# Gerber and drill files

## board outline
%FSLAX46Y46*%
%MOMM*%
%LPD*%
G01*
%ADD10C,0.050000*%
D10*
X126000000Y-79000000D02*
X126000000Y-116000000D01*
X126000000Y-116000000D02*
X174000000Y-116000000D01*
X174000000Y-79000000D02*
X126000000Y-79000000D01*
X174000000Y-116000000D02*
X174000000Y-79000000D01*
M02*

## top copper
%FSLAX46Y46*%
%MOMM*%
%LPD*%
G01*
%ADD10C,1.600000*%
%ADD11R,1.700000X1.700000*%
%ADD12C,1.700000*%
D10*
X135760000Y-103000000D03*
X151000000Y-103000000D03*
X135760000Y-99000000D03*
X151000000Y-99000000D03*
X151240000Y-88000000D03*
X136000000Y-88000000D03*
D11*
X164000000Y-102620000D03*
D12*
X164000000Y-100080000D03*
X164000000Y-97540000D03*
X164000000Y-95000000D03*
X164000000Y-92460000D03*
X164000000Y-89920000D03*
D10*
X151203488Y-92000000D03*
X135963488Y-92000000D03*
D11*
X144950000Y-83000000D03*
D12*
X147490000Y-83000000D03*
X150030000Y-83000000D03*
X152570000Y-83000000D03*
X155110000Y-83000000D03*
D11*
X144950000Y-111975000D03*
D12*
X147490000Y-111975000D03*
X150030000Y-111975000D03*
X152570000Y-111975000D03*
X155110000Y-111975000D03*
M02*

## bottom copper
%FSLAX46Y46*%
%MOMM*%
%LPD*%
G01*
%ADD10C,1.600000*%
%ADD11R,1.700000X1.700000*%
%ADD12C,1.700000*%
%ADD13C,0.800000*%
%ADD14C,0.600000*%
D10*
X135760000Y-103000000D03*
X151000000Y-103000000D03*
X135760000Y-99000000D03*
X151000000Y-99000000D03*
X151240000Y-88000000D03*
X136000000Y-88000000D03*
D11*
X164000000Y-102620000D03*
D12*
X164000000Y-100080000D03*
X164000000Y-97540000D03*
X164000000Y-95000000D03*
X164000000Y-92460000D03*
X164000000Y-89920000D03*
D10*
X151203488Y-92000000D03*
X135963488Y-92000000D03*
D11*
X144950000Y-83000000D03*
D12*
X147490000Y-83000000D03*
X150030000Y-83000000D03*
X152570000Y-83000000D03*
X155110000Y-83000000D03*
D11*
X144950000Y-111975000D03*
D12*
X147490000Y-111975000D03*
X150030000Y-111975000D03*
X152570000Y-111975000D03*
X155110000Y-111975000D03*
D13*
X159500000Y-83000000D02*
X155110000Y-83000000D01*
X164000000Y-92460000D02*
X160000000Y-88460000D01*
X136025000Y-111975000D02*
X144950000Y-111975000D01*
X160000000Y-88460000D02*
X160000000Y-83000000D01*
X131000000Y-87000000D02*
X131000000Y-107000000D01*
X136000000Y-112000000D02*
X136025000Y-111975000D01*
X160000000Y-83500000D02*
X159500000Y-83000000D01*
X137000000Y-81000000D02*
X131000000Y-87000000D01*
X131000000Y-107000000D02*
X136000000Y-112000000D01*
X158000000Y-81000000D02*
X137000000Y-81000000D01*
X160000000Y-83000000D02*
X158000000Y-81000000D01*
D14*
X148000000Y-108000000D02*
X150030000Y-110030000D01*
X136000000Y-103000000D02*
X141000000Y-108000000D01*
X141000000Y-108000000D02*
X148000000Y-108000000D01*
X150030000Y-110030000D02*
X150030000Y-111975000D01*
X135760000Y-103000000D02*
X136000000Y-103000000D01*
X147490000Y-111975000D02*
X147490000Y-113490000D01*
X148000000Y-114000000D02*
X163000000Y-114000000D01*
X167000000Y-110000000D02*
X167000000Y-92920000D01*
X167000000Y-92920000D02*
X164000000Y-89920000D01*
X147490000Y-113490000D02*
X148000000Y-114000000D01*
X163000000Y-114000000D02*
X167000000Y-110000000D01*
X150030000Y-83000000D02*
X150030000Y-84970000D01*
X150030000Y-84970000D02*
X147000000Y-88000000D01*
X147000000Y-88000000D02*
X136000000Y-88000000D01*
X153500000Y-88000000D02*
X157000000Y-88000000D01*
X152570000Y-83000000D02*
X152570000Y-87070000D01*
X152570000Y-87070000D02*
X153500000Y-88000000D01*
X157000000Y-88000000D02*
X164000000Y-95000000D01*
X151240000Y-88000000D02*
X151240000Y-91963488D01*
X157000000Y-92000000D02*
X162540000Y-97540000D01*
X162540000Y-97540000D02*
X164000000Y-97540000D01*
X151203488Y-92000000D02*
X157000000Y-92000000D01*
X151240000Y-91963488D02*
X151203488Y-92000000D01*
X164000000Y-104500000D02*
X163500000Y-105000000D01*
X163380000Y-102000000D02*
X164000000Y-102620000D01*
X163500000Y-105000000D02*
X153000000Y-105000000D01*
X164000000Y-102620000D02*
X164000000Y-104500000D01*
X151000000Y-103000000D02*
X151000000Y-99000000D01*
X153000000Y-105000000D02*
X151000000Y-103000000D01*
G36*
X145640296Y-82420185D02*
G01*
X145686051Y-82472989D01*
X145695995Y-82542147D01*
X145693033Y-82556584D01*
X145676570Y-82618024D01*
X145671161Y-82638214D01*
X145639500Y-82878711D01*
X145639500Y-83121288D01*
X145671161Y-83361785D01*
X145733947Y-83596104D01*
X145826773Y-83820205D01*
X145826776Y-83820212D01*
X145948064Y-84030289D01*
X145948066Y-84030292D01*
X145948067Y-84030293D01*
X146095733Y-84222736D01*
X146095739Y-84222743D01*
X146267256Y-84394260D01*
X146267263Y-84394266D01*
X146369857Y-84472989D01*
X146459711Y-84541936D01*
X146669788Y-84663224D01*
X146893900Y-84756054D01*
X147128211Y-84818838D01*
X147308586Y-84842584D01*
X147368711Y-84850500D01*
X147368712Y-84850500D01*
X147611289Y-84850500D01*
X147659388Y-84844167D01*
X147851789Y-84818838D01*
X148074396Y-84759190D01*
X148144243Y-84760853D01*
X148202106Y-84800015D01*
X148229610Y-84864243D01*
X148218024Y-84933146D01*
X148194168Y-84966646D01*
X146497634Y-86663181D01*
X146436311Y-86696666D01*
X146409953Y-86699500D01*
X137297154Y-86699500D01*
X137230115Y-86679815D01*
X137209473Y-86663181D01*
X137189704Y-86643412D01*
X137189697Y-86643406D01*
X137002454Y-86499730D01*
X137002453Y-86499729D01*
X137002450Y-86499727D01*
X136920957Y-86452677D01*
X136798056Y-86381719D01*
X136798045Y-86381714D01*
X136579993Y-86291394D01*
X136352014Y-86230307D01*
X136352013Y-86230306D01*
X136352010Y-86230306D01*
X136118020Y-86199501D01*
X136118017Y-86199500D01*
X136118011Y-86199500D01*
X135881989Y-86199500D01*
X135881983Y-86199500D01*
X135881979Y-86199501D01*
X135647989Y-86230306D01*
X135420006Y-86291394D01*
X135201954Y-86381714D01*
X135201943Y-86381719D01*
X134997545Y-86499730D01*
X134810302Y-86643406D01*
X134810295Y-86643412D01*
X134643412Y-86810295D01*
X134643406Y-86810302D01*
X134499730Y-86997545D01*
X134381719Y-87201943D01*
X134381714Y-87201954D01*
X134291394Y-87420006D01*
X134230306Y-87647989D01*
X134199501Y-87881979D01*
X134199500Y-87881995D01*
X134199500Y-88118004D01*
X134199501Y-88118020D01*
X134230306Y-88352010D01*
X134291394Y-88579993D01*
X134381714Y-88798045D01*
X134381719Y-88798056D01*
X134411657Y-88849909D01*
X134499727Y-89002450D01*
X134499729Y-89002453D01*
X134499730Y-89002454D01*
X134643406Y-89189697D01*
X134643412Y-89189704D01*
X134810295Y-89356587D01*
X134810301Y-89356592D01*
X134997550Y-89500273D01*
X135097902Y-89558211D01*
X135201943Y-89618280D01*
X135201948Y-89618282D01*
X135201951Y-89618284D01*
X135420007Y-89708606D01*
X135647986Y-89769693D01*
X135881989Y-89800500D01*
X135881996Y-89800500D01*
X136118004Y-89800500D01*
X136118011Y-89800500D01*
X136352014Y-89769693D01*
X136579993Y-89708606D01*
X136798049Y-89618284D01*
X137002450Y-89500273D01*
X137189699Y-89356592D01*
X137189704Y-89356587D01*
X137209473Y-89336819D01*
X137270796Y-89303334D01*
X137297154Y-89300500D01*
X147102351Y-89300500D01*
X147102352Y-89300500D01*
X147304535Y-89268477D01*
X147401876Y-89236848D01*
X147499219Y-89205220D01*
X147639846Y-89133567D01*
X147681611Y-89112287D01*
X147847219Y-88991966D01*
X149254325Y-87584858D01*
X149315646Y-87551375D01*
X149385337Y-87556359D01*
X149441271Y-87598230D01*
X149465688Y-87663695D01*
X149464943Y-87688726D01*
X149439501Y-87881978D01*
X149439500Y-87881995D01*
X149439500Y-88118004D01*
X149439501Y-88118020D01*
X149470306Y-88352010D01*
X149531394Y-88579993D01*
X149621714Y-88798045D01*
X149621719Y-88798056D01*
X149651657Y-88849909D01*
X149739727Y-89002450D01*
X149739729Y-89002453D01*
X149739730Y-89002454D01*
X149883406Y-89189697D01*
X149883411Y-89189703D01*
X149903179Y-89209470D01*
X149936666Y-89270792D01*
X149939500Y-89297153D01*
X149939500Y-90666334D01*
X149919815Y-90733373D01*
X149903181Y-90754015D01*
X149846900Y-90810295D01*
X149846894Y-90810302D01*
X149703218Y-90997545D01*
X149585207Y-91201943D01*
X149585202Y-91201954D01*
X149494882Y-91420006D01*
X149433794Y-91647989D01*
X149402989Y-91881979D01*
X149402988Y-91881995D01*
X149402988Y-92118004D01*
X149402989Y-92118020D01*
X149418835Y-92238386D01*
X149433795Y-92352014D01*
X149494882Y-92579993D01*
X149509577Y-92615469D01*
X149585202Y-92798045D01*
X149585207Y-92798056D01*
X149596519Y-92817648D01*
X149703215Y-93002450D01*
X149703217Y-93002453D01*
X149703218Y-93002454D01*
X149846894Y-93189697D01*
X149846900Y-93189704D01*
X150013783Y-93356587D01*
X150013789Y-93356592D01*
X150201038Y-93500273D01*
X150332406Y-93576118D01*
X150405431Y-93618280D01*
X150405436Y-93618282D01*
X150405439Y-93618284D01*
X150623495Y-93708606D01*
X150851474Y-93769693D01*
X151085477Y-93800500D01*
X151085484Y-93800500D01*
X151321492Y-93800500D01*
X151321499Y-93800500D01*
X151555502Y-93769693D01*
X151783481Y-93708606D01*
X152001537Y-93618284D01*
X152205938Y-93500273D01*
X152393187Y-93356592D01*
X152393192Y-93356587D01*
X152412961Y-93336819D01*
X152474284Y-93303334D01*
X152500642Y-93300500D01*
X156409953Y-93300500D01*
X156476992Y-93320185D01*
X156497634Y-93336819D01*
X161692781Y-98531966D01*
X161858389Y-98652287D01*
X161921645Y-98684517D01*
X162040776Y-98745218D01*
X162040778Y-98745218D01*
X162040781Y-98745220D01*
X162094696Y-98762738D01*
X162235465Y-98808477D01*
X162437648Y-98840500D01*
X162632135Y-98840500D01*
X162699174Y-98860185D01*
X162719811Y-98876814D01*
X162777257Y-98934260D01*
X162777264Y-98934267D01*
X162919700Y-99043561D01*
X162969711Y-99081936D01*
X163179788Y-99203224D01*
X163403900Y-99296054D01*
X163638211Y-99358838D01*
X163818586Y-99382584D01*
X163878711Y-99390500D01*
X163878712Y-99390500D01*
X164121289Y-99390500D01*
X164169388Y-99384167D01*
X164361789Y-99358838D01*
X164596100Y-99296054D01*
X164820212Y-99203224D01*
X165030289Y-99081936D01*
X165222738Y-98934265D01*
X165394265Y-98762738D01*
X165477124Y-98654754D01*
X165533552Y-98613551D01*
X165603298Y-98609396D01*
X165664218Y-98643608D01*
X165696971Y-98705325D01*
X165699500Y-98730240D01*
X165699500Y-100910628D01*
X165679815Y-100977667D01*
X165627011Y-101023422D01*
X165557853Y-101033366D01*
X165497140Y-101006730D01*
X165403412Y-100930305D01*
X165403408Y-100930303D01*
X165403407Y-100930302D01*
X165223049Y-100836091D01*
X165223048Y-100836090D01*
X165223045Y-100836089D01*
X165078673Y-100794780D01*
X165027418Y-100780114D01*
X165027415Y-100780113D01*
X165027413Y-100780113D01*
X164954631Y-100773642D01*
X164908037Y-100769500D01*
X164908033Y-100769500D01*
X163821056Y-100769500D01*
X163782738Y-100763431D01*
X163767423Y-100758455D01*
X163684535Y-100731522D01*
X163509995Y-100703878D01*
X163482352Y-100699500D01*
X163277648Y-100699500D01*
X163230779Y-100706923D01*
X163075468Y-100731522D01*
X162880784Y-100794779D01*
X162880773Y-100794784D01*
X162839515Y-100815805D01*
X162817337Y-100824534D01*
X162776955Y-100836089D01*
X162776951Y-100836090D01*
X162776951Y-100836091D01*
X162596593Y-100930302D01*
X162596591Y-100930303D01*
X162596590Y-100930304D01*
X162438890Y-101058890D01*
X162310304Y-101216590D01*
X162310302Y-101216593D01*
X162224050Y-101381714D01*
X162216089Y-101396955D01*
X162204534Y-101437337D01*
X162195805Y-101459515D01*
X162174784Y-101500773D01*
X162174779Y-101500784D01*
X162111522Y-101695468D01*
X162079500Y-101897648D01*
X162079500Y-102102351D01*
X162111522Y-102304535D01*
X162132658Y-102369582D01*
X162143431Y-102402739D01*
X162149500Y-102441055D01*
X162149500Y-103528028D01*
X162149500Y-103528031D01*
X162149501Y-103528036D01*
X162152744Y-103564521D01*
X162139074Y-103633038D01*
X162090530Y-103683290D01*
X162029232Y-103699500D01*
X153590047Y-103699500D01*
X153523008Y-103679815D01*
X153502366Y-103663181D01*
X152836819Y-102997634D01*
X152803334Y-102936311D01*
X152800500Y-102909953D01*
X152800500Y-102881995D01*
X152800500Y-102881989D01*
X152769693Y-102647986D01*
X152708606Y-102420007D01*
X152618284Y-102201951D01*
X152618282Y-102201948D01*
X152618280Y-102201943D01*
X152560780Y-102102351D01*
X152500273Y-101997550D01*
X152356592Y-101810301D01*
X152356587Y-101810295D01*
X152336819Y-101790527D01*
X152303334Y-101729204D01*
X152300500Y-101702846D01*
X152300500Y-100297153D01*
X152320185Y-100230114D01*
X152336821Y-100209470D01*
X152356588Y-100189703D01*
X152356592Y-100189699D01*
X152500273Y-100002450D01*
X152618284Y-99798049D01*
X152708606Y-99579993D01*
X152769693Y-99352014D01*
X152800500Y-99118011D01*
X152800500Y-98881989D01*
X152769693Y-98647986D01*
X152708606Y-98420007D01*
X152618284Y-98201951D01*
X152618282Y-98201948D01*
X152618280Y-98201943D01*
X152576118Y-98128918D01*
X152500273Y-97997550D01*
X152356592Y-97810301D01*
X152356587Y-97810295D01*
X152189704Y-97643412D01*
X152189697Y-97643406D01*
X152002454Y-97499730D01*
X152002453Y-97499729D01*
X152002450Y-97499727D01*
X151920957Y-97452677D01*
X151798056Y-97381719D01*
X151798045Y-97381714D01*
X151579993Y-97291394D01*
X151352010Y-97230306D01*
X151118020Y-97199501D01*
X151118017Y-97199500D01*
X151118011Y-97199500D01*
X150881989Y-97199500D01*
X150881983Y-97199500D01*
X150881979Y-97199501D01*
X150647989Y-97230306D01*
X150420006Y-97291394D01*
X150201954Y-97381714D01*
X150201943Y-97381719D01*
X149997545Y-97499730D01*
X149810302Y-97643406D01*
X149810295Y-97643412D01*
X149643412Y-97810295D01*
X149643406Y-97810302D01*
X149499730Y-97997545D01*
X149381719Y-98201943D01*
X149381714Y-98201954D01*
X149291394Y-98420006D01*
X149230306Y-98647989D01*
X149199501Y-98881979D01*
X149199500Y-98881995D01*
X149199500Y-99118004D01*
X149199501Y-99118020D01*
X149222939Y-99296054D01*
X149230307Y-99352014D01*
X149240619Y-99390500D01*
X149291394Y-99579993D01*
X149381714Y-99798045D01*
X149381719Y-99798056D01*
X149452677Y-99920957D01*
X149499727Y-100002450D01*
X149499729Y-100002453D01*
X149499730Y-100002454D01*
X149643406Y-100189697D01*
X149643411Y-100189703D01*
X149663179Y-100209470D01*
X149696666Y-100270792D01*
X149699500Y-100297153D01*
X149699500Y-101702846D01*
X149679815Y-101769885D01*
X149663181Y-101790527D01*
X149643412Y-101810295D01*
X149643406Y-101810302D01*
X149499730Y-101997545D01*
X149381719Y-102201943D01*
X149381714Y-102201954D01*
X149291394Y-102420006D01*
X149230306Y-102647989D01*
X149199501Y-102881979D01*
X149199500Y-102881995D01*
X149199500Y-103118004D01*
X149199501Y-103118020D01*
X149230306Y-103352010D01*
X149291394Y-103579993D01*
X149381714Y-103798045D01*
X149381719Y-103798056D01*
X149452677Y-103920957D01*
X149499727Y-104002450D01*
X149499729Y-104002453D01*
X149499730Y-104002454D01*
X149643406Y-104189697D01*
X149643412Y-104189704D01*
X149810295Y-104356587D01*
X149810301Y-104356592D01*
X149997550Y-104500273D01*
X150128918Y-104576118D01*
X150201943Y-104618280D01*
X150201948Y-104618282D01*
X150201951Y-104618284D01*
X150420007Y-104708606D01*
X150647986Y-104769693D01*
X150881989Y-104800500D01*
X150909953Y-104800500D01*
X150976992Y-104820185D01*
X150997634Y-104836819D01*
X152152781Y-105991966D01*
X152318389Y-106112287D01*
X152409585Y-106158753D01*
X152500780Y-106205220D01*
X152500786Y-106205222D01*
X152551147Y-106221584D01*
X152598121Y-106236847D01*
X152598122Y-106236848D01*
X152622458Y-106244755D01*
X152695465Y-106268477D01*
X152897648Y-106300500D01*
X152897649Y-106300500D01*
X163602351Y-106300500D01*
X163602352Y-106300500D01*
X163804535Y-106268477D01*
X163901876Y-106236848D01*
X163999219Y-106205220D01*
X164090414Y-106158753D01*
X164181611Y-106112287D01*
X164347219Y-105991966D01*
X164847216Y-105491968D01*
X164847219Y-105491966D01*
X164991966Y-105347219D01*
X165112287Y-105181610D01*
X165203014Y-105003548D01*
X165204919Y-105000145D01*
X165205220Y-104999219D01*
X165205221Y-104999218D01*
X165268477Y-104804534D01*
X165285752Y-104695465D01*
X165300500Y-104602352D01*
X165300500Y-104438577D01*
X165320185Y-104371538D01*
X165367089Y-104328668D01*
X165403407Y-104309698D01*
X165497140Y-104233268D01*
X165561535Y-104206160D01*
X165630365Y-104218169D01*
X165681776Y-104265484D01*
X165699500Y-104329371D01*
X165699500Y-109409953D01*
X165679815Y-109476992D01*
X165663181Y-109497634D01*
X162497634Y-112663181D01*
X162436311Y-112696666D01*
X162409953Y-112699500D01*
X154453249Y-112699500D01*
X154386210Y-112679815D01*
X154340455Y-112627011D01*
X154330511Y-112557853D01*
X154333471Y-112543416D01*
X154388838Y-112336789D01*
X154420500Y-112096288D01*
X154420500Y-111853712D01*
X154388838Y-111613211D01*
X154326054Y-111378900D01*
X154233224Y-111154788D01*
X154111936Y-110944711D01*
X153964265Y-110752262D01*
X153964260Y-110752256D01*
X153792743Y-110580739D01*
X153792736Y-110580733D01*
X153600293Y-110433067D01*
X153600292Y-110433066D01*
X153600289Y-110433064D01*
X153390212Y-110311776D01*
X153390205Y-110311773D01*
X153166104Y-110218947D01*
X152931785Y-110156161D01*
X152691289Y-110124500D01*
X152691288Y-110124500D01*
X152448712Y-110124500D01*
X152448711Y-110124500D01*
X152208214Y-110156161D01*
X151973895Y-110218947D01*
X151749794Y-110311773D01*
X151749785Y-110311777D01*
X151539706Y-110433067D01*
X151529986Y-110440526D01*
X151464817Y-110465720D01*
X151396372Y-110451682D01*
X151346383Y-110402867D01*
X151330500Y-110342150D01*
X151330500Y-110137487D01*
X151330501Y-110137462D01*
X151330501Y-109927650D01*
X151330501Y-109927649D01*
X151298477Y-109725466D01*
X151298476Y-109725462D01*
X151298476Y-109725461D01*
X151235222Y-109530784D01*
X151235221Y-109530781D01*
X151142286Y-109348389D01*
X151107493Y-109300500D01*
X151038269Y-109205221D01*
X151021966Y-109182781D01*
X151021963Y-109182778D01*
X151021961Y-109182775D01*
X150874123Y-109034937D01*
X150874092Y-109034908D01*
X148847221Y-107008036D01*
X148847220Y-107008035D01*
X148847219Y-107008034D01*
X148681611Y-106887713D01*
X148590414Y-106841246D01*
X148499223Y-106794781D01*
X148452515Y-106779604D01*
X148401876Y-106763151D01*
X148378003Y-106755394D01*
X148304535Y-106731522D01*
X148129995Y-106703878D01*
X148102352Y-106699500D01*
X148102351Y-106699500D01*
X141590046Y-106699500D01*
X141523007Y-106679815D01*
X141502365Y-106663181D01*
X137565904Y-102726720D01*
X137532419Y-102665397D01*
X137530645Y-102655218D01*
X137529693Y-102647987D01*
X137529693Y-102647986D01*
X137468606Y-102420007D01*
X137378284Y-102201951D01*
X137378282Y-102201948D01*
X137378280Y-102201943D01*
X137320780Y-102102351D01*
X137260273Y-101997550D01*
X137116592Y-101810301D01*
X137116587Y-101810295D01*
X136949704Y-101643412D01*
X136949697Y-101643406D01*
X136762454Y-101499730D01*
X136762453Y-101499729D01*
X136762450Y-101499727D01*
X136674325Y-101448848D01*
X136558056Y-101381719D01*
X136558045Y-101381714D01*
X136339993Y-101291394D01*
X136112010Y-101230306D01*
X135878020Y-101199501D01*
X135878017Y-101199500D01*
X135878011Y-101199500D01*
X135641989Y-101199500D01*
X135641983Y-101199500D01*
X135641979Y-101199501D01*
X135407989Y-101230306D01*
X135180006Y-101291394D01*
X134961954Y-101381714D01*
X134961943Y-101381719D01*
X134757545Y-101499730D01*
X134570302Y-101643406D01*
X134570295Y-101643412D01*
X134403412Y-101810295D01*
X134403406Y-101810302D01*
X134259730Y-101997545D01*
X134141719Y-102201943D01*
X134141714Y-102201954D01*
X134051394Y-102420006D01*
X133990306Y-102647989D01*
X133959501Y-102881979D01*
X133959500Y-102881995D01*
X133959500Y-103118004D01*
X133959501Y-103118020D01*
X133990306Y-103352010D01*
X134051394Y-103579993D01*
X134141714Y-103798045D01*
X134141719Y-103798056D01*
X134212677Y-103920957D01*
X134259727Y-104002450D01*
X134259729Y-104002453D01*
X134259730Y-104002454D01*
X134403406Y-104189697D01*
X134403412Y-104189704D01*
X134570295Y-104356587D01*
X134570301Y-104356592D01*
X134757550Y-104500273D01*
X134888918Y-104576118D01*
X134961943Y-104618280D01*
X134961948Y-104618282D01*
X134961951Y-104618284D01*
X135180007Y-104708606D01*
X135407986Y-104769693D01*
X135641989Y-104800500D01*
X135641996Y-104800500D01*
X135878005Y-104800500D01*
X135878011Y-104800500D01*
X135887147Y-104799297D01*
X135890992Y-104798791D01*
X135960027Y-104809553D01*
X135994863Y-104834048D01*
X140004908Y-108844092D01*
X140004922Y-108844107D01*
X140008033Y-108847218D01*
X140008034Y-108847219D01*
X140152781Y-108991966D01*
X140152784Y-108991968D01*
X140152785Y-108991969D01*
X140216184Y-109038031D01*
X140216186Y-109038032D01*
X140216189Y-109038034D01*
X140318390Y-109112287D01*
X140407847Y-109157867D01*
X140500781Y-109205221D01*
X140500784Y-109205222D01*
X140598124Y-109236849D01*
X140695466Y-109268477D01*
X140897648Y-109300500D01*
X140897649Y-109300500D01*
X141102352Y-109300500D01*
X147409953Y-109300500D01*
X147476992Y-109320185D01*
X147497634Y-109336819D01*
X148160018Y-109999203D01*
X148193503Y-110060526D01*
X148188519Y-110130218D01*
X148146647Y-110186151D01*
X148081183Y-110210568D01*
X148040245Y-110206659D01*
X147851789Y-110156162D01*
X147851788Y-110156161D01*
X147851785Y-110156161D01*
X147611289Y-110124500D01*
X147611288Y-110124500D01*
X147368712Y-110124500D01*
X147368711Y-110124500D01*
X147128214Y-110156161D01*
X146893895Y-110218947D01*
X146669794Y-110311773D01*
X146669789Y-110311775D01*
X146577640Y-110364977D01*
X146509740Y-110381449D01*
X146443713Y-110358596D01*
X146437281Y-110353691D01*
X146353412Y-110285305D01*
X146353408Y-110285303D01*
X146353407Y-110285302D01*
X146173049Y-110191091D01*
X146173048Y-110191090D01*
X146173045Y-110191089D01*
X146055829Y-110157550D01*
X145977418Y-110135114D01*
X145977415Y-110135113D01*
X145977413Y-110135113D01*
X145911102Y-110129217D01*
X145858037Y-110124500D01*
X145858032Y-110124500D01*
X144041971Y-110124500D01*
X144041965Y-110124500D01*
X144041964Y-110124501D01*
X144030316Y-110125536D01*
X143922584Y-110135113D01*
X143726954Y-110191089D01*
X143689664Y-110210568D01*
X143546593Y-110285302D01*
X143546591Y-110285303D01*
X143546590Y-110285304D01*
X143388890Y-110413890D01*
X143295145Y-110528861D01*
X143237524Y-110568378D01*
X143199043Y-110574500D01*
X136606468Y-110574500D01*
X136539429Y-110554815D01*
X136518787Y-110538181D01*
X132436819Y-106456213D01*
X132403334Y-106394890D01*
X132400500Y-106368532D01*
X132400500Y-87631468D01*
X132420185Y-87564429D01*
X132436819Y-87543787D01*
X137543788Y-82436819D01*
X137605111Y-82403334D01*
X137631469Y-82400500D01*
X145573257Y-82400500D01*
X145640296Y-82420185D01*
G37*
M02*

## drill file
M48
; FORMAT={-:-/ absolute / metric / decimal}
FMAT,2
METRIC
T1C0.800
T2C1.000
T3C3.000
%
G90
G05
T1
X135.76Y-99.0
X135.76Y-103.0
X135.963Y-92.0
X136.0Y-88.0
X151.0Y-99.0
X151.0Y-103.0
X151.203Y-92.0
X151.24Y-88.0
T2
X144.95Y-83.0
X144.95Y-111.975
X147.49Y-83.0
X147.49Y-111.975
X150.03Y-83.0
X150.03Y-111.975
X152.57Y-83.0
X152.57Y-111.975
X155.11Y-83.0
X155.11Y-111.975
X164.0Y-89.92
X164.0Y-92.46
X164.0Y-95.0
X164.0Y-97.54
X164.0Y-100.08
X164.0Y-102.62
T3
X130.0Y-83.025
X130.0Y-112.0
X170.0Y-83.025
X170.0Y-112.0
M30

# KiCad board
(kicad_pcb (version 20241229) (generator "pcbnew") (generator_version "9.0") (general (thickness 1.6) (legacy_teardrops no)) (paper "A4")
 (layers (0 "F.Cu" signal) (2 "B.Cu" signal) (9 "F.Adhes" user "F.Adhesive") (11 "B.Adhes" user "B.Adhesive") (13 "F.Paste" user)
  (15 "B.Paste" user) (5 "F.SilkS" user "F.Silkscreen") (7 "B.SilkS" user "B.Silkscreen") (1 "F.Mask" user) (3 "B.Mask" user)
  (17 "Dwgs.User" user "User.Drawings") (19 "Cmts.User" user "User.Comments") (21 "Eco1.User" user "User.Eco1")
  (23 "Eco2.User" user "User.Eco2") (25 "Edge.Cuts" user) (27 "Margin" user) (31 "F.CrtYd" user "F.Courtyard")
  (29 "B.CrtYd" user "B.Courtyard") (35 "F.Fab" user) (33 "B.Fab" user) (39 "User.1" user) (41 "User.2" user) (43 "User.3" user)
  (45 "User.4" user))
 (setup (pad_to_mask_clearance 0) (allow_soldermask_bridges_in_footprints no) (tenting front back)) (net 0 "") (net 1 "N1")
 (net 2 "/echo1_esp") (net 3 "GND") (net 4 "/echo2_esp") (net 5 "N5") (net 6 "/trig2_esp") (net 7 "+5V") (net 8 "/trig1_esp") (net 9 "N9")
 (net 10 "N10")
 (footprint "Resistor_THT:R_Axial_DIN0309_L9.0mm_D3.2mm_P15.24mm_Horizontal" (layer "F.Cu") (at 135.76 103)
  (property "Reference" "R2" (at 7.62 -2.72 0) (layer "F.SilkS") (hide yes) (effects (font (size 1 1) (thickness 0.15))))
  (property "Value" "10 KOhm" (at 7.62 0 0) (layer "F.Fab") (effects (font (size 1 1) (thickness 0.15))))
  (pad "1" thru_hole circle (at 0 0) (size 1.6 1.6) (drill 0.8) (layers "*.Cu" "*.Mask") (remove_unused_layers no) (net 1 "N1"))
  (pad "2" thru_hole circle (at 15.24 0) (size 1.6 1.6) (drill 0.8) (layers "*.Cu" "*.Mask") (remove_unused_layers no) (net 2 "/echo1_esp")))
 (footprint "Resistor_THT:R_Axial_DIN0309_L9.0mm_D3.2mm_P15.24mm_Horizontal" (layer "F.Cu") (at 135.76 99)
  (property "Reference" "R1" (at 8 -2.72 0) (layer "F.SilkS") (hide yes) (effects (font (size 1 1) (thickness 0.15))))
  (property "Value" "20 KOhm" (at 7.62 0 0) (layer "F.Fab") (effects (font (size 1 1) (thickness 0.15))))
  (pad "1" thru_hole circle (at 0 0) (size 1.6 1.6) (drill 0.8) (layers "*.Cu" "*.Mask") (remove_unused_layers no) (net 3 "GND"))
  (pad "2" thru_hole circle (at 15.24 0) (size 1.6 1.6) (drill 0.8) (layers "*.Cu" "*.Mask") (remove_unused_layers no) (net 2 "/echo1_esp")))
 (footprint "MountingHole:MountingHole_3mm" (layer "F.Cu") (at 130 112)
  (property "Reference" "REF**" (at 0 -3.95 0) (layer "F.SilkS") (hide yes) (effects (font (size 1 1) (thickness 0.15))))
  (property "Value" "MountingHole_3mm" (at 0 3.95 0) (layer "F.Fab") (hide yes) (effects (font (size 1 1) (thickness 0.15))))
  (pad "" np_thru_hole circle (at 0 0) (size 3 3) (drill 3) (layers "*.Cu" "*.Mask")))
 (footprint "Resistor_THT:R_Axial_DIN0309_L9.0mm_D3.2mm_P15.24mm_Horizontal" (layer "F.Cu") (at 151.24 88 180)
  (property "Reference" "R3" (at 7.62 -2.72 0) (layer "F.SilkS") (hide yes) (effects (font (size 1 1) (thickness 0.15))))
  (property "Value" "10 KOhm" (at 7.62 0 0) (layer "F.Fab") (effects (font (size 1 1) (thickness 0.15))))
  (pad "1" thru_hole circle (at 0 0 180) (size 1.6 1.6) (drill 0.8) (layers "*.Cu" "*.Mask") (remove_unused_layers no) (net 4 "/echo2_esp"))
  (pad "2" thru_hole circle (at 15.24 0 180) (size 1.6 1.6) (drill 0.8) (layers "*.Cu" "*.Mask") (remove_unused_layers no) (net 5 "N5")))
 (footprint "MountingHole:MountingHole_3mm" (layer "F.Cu") (at 170 112)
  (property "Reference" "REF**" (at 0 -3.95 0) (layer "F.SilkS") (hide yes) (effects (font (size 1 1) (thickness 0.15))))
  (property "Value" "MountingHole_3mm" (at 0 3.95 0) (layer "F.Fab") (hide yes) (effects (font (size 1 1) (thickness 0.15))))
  (pad "" np_thru_hole circle (at 0 0) (size 3 3) (drill 3) (layers "*.Cu" "*.Mask")))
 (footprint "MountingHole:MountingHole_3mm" (layer "F.Cu") (at 130 83.025)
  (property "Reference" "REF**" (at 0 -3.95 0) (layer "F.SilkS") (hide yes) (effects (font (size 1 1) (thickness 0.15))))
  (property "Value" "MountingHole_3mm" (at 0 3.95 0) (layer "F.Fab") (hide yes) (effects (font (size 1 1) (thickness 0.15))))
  (pad "" np_thru_hole circle (at 0 0) (size 3 3) (drill 3) (layers "*.Cu" "*.Mask")))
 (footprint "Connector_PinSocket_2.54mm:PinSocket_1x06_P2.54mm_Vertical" (layer "F.Cu") (at 164 102.62 180)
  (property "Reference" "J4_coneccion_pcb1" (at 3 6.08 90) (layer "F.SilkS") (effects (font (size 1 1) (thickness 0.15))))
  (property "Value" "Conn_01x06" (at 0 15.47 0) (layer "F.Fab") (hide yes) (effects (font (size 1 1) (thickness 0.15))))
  (pad "1" thru_hole rect (at 0 0 180) (size 1.7 1.7) (drill 1) (layers "*.Cu" "*.Mask") (remove_unused_layers no) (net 2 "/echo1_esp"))
  (pad "2" thru_hole circle (at 0 2.54 180) (size 1.7 1.7) (drill 1) (layers "*.Cu" "*.Mask") (remove_unused_layers no) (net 3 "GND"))
  (pad "3" thru_hole circle (at 0 5.08 180) (size 1.7 1.7) (drill 1) (layers "*.Cu" "*.Mask") (remove_unused_layers no) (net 4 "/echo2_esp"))
  (pad "4" thru_hole circle (at 0 7.62 180) (size 1.7 1.7) (drill 1) (layers "*.Cu" "*.Mask") (remove_unused_layers no) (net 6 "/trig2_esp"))
  (pad "5" thru_hole circle (at 0 10.16 180) (size 1.7 1.7) (drill 1) (layers "*.Cu" "*.Mask") (remove_unused_layers no) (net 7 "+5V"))
  (pad "6" thru_hole circle (at 0 12.7 180) (size 1.7 1.7) (drill 1) (layers "*.Cu" "*.Mask") (remove_unused_layers no) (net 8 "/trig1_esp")))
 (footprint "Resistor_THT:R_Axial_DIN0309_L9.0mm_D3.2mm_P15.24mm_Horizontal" (layer "F.Cu") (at 151.203488 92 180)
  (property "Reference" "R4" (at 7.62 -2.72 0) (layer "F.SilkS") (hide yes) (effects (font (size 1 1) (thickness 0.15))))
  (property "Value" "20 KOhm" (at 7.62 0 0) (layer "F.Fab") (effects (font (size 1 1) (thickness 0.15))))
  (pad "1" thru_hole circle (at 0 0 180) (size 1.6 1.6) (drill 0.8) (layers "*.Cu" "*.Mask") (remove_unused_layers no) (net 4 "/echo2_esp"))
  (pad "2" thru_hole circle (at 15.24 0 180) (size 1.6 1.6) (drill 0.8) (layers "*.Cu" "*.Mask") (remove_unused_layers no) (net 3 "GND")))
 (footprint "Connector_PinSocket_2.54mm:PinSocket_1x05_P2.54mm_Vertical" (layer "F.Cu") (at 144.95 83 90)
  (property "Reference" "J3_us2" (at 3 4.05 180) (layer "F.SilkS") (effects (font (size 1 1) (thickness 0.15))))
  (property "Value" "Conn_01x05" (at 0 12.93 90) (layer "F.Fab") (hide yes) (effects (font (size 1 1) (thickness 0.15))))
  (pad "1" thru_hole rect (at 0 0 90) (size 1.7 1.7) (drill 1) (layers "*.Cu" "*.Mask") (remove_unused_layers no) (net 3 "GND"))
  (pad "2" thru_hole circle (at 0 2.54 90) (size 1.7 1.7) (drill 1) (layers "*.Cu" "*.Mask") (remove_unused_layers no) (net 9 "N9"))
  (pad "3" thru_hole circle (at 0 5.08 90) (size 1.7 1.7) (drill 1) (layers "*.Cu" "*.Mask") (remove_unused_layers no) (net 5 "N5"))
  (pad "4" thru_hole circle (at 0 7.62 90) (size 1.7 1.7) (drill 1) (layers "*.Cu" "*.Mask") (remove_unused_layers no) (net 6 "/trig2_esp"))
  (pad "5" thru_hole circle (at 0 10.16 90) (size 1.7 1.7) (drill 1) (layers "*.Cu" "*.Mask") (remove_unused_layers no) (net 7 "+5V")))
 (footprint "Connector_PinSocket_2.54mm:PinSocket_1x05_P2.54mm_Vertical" (layer "F.Cu") (at 144.95 111.975 90)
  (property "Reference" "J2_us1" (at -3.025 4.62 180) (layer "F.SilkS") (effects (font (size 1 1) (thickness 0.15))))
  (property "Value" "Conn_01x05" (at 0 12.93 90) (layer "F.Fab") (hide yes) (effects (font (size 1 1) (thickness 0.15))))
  (pad "1" thru_hole rect (at 0 0 90) (size 1.7 1.7) (drill 1) (layers "*.Cu" "*.Mask") (remove_unused_layers no) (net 7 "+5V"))
  (pad "2" thru_hole circle (at 0 2.54 90) (size 1.7 1.7) (drill 1) (layers "*.Cu" "*.Mask") (remove_unused_layers no) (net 8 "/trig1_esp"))
  (pad "3" thru_hole circle (at 0 5.08 90) (size 1.7 1.7) (drill 1) (layers "*.Cu" "*.Mask") (remove_unused_layers no) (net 1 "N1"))
  (pad "4" thru_hole circle (at 0 7.62 90) (size 1.7 1.7) (drill 1) (layers "*.Cu" "*.Mask") (remove_unused_layers no) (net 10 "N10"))
  (pad "5" thru_hole circle (at 0 10.16 90) (size 1.7 1.7) (drill 1) (layers "*.Cu" "*.Mask") (remove_unused_layers no) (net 3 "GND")))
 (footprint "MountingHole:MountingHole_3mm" (layer "F.Cu") (at 170 83.025)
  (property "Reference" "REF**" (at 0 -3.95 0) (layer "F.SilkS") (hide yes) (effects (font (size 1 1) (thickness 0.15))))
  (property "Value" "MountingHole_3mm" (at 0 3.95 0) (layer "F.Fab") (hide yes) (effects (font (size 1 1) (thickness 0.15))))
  (pad "" np_thru_hole circle (at 0 0) (size 3 3) (drill 3) (layers "*.Cu" "*.Mask")))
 (gr_line (start 126 79) (end 126 116) (stroke (width 0.05) (type default)) (locked yes) (layer "Edge.Cuts"))
 (gr_line (start 126 116) (end 174 116) (stroke (width 0.05) (type default)) (locked yes) (layer "Edge.Cuts"))
 (gr_line (start 174 79) (end 126 79) (stroke (width 0.05) (type default)) (locked yes) (layer "Edge.Cuts"))
 (gr_line (start 174 116) (end 174 79) (stroke (width 0.05) (type default)) (locked yes) (layer "Edge.Cuts"))
 (segment (start 159.5 83) (end 155.11 83) (width 0.8) (layer "B.Cu") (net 7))
 (segment (start 164 92.46) (end 160 88.46) (width 0.8) (layer "B.Cu") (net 7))
 (segment (start 136.025 111.975) (end 144.95 111.975) (width 0.8) (layer "B.Cu") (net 7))
 (segment (start 160 88.46) (end 160 83) (width 0.8) (layer "B.Cu") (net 7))
 (segment (start 131 87) (end 131 107) (width 0.8) (layer "B.Cu") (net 7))
 (segment (start 136 112) (end 136.025 111.975) (width 0.8) (layer "B.Cu") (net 7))
 (segment (start 160 83.5) (end 159.5 83) (width 0.8) (layer "B.Cu") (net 7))
 (segment (start 137 81) (end 131 87) (width 0.8) (layer "B.Cu") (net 7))
 (segment (start 131 107) (end 136 112) (width 0.8) (layer "B.Cu") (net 7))
 (segment (start 158 81) (end 137 81) (width 0.8) (layer "B.Cu") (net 7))
 (segment (start 160 83) (end 158 81) (width 0.8) (layer "B.Cu") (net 7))
 (segment (start 148 108) (end 150.03 110.03) (width 0.6) (layer "B.Cu") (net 1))
 (segment (start 136 103) (end 141 108) (width 0.6) (layer "B.Cu") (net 1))
 (segment (start 141 108) (end 148 108) (width 0.6) (layer "B.Cu") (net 1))
 (segment (start 150.03 110.03) (end 150.03 111.975) (width 0.6) (layer "B.Cu") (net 1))
 (segment (start 135.76 103) (end 136 103) (width 0.6) (layer "B.Cu") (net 1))
 (segment (start 147.49 111.975) (end 147.49 113.49) (width 0.6) (layer "B.Cu") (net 8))
 (segment (start 148 114) (end 163 114) (width 0.6) (layer "B.Cu") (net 8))
 (segment (start 167 110) (end 167 92.92) (width 0.6) (layer "B.Cu") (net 8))
 (segment (start 167 92.92) (end 164 89.92) (width 0.6) (layer "B.Cu") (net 8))
 (segment (start 147.49 113.49) (end 148 114) (width 0.6) (layer "B.Cu") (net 8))
 (segment (start 163 114) (end 167 110) (width 0.6) (layer "B.Cu") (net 8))
 (segment (start 150.03 83) (end 150.03 84.97) (width 0.6) (layer "B.Cu") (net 5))
 (segment (start 150.03 84.97) (end 147 88) (width 0.6) (layer "B.Cu") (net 5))
 (segment (start 147 88) (end 136 88) (width 0.6) (layer "B.Cu") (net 5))
 (segment (start 153.5 88) (end 157 88) (width 0.6) (layer "B.Cu") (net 6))
 (segment (start 152.57 83) (end 152.57 87.07) (width 0.6) (layer "B.Cu") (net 6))
 (segment (start 152.57 87.07) (end 153.5 88) (width 0.6) (layer "B.Cu") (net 6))
 (segment (start 157 88) (end 164 95) (width 0.6) (layer "B.Cu") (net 6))
 (segment (start 151.24 88) (end 151.24 91.963488) (width 0.6) (layer "B.Cu") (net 4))
 (segment (start 157 92) (end 162.54 97.54) (width 0.6) (layer "B.Cu") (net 4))
 (segment (start 162.54 97.54) (end 164 97.54) (width 0.6) (layer "B.Cu") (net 4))
 (segment (start 151.203488 92) (end 157 92) (width 0.6) (layer "B.Cu") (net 4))
 (segment (start 151.24 91.963488) (end 151.203488 92) (width 0.6) (layer "B.Cu") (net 4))
 (segment (start 164 104.5) (end 163.5 105) (width 0.6) (layer "B.Cu") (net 2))
 (segment (start 163.38 102) (end 164 102.62) (width 0.6) (layer "B.Cu") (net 2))
 (segment (start 163.5 105) (end 153 105) (width 0.6) (layer "B.Cu") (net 2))
 (segment (start 164 102.62) (end 164 104.5) (width 0.6) (layer "B.Cu") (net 2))
 (segment (start 151 103) (end 151 99) (width 0.6) (layer "B.Cu") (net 2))
 (segment (start 153 105) (end 151 103) (width 0.6) (layer "B.Cu") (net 2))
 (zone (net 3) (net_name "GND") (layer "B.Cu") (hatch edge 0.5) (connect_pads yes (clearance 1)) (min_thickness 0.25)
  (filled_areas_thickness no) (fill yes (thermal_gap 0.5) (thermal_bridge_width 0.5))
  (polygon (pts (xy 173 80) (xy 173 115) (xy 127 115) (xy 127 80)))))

